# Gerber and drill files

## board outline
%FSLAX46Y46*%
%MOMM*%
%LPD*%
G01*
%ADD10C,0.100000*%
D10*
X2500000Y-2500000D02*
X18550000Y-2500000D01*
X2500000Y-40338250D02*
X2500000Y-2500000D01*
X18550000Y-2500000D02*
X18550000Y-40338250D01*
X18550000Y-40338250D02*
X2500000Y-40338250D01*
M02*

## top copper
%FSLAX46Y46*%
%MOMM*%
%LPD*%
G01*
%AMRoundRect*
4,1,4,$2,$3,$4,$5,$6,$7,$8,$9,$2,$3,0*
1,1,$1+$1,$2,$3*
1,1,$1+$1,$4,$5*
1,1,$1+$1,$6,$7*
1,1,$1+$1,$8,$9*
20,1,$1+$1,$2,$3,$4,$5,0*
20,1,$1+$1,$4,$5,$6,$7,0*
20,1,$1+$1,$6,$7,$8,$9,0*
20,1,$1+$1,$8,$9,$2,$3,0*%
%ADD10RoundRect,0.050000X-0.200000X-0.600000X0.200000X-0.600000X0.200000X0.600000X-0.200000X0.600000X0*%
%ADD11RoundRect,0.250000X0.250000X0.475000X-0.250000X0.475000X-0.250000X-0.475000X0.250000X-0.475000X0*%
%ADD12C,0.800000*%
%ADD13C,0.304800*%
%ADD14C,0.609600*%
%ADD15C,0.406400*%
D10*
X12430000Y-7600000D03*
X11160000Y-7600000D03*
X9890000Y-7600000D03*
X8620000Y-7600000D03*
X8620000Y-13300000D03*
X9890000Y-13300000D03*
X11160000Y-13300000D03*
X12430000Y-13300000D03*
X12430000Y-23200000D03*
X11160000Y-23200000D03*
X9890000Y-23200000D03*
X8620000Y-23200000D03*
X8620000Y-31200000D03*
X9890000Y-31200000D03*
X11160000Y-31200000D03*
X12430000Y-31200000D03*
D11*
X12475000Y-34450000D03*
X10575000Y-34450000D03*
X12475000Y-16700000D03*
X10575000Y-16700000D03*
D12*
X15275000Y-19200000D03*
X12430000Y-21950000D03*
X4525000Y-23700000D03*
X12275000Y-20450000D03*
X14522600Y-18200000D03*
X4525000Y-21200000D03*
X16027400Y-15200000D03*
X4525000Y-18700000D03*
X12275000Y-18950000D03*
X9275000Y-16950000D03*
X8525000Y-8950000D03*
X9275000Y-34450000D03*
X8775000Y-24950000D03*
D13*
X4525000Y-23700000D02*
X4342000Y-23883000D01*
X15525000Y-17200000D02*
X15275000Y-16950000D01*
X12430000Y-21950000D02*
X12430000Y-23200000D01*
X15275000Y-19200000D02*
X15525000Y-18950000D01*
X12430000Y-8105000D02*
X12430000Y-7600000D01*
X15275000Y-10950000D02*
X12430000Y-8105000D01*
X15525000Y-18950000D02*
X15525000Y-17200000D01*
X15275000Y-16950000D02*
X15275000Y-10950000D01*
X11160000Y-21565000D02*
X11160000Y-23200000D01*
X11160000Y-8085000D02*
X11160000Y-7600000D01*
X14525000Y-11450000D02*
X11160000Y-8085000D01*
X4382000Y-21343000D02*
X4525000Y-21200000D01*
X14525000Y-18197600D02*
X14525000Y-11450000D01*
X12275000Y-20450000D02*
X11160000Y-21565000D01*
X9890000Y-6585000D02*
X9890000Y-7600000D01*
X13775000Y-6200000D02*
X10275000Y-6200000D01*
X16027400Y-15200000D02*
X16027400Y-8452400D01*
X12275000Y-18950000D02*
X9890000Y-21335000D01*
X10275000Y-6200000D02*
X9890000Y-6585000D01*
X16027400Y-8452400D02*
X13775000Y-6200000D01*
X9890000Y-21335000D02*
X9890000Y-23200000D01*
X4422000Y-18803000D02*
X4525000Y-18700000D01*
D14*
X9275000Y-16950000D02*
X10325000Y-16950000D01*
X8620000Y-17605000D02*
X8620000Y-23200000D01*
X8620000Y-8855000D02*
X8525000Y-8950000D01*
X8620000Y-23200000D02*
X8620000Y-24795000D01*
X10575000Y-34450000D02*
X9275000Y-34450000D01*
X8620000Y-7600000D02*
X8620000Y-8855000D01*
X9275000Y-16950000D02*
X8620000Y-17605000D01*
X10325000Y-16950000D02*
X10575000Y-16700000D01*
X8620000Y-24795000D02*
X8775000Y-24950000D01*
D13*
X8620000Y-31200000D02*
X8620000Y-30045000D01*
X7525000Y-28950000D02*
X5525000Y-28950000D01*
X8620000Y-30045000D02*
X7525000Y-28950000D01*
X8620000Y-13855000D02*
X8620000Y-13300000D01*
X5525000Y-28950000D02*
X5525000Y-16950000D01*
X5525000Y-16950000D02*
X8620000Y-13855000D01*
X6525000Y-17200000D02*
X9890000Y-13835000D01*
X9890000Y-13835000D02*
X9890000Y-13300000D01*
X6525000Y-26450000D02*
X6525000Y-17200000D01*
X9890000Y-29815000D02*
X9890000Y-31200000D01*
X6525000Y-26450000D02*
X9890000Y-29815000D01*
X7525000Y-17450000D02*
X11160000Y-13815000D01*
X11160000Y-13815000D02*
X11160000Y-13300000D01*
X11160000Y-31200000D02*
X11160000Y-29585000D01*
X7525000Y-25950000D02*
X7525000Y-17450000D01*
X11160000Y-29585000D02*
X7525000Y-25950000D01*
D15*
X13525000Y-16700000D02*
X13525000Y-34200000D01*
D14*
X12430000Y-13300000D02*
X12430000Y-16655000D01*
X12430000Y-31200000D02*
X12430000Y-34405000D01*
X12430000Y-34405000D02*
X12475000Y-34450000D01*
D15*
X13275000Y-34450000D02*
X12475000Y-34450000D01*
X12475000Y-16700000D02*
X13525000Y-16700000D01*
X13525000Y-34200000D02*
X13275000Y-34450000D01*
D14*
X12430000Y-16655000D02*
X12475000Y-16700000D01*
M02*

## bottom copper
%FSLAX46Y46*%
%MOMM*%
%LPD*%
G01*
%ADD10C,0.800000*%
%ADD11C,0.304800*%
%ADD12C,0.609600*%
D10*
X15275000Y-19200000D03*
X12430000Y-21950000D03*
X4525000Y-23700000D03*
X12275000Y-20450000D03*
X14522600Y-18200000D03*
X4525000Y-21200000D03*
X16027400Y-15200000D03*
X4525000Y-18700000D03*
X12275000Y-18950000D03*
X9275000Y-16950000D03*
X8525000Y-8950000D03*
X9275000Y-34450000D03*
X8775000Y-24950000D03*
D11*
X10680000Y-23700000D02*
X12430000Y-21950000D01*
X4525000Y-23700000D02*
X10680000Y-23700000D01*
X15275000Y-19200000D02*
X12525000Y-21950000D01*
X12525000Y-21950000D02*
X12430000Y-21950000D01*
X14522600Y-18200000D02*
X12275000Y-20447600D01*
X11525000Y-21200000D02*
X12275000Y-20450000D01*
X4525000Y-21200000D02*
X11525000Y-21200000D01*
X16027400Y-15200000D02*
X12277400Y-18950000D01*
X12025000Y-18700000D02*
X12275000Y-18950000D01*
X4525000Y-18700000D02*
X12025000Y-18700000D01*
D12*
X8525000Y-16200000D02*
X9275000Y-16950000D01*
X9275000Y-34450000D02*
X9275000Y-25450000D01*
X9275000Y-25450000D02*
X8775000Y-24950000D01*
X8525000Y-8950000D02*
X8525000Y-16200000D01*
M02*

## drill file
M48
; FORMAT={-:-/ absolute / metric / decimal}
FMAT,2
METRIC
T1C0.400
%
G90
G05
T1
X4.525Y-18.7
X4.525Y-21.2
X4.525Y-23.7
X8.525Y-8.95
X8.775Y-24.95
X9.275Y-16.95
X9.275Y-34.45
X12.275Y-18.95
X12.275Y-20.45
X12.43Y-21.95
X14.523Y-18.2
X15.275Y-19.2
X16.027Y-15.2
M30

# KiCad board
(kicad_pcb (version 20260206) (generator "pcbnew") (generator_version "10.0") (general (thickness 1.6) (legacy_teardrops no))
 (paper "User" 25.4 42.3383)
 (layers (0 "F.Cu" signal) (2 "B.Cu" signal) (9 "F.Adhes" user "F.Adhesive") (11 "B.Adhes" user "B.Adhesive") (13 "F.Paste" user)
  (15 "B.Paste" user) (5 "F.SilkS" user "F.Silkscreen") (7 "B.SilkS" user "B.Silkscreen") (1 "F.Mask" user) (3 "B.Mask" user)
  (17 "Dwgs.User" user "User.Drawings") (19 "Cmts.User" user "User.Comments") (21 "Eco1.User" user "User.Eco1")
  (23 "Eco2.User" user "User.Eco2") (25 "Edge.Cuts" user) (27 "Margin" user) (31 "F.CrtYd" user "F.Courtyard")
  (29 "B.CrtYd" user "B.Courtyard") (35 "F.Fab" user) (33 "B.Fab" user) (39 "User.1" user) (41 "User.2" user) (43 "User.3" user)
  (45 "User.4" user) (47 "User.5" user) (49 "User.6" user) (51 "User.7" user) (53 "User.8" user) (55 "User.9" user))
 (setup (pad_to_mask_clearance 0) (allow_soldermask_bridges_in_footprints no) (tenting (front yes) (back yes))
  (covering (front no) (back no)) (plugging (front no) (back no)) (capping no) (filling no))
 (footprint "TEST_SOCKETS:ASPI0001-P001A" (layer "F.Cu") (at 10.525 10.45)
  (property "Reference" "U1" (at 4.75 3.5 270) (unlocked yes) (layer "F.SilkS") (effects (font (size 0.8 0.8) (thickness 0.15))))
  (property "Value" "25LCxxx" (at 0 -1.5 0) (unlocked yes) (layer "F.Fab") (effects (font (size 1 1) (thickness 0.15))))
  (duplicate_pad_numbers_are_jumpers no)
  (pad "1" smd roundrect (at 1.905 -2.85) (size 0.5 1.3) (layers "F.Cu" "F.Mask" "F.Paste") (roundrect_rratio 0.1) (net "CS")
   (thermal_bridge_angle 45))
  (pad "2" smd roundrect (at 0.635 -2.85) (size 0.5 1.3) (layers "F.Cu" "F.Mask" "F.Paste") (roundrect_rratio 0.1) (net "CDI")
   (thermal_bridge_angle 45))
  (pad "3" smd roundrect (at -0.635 -2.85) (size 0.5 1.3) (layers "F.Cu" "F.Mask" "F.Paste") (roundrect_rratio 0.1) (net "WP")
   (thermal_bridge_angle 45))
  (pad "4" smd roundrect (at -1.905 -2.85) (size 0.5 1.3) (layers "F.Cu" "F.Mask" "F.Paste") (roundrect_rratio 0.1) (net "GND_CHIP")
   (thermal_bridge_angle 45))
  (pad "5" smd roundrect (at -1.905 2.85) (size 0.5 1.3) (layers "F.Cu" "F.Mask" "F.Paste") (roundrect_rratio 0.1) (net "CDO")
   (thermal_bridge_angle 45))
  (pad "6" smd roundrect (at -0.635 2.85) (size 0.5 1.3) (layers "F.Cu" "F.Mask" "F.Paste") (roundrect_rratio 0.1) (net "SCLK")
   (thermal_bridge_angle 45))
  (pad "7" smd roundrect (at 0.635 2.85) (size 0.5 1.3) (layers "F.Cu" "F.Mask" "F.Paste") (roundrect_rratio 0.1) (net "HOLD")
   (thermal_bridge_angle 45))
  (pad "8" smd roundrect (at 1.905 2.85) (size 0.5 1.3) (layers "F.Cu" "F.Mask" "F.Paste") (roundrect_rratio 0.1) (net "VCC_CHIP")
   (thermal_bridge_angle 45)))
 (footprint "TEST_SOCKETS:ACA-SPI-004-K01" (layer "F.Cu") (at 10.525 27.2)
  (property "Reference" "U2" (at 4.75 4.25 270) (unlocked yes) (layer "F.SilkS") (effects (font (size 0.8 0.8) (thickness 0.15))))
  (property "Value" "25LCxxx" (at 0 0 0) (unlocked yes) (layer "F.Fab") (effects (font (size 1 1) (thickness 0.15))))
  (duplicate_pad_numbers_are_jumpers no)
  (pad "1" smd roundrect (at 1.905 -4) (size 0.5 1.3) (layers "F.Cu" "F.Mask" "F.Paste") (roundrect_rratio 0.1) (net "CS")
   (thermal_bridge_angle 45))
  (pad "2" smd roundrect (at 0.635 -4) (size 0.5 1.3) (layers "F.Cu" "F.Mask" "F.Paste") (roundrect_rratio 0.1) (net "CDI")
   (thermal_bridge_angle 45))
  (pad "3" smd roundrect (at -0.635 -4) (size 0.5 1.3) (layers "F.Cu" "F.Mask" "F.Paste") (roundrect_rratio 0.1) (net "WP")
   (thermal_bridge_angle 45))
  (pad "4" smd roundrect (at -1.905 -4) (size 0.5 1.3) (layers "F.Cu" "F.Mask" "F.Paste") (roundrect_rratio 0.1) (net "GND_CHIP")
   (thermal_bridge_angle 45))
  (pad "5" smd roundrect (at -1.905 4) (size 0.5 1.3) (layers "F.Cu" "F.Mask" "F.Paste") (roundrect_rratio 0.1) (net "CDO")
   (thermal_bridge_angle 45))
  (pad "6" smd roundrect (at -0.635 4) (size 0.5 1.3) (layers "F.Cu" "F.Mask" "F.Paste") (roundrect_rratio 0.1) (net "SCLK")
   (thermal_bridge_angle 45))
  (pad "7" smd roundrect (at 0.635 4) (size 0.5 1.3) (layers "F.Cu" "F.Mask" "F.Paste") (roundrect_rratio 0.1) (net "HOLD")
   (thermal_bridge_angle 45))
  (pad "8" smd roundrect (at 1.905 4) (size 0.5 1.3) (layers "F.Cu" "F.Mask" "F.Paste") (roundrect_rratio 0.1) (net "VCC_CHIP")
   (thermal_bridge_angle 45)))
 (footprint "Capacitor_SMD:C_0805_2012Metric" (layer "F.Cu") (at 11.525 34.45 180)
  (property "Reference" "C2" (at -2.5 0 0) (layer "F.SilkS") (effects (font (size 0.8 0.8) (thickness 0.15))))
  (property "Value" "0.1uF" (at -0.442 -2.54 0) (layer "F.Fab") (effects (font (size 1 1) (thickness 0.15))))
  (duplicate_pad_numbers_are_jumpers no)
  (pad "1" smd roundrect (at -0.95 0 180) (size 1 1.45) (layers "F.Cu" "F.Mask" "F.Paste") (roundrect_rratio 0.25) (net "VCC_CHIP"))
  (pad "2" smd roundrect (at 0.95 0 180) (size 1 1.45) (layers "F.Cu" "F.Mask" "F.Paste") (roundrect_rratio 0.25) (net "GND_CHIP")))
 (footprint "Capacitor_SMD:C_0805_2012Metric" (layer "F.Cu") (at 11.525 16.7 180)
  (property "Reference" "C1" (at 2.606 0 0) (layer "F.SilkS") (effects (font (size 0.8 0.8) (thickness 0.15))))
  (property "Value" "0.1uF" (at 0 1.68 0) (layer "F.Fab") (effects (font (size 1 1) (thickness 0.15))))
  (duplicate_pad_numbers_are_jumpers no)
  (pad "1" smd roundrect (at -0.95 0 180) (size 1 1.45) (layers "F.Cu" "F.Mask" "F.Paste") (roundrect_rratio 0.25) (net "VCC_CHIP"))
  (pad "2" smd roundrect (at 0.95 0 180) (size 1 1.45) (layers "F.Cu" "F.Mask" "F.Paste") (roundrect_rratio 0.25) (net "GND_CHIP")))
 (gr_line (start 2.5 2.5) (end 18.55 2.5) (stroke (width 0.1) (type default)) (layer "Edge.Cuts"))
 (gr_line (start 2.5 40.33825) (end 2.5 2.5) (stroke (width 0.1) (type default)) (layer "Edge.Cuts"))
 (gr_line (start 18.55 2.5) (end 18.55 40.33825) (stroke (width 0.1) (type default)) (layer "Edge.Cuts"))
 (gr_line (start 18.55 40.33825) (end 2.5 40.33825) (stroke (width 0.1) (type default)) (layer "Edge.Cuts"))
 (segment (start 4.525 23.7) (end 4.342 23.883) (width 0.3048) (layer "F.Cu") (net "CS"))
 (segment (start 15.525 17.2) (end 15.275 16.95) (width 0.3048) (layer "F.Cu") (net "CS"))
 (segment (start 12.43 21.95) (end 12.43 23.2) (width 0.3048) (layer "F.Cu") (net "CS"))
 (segment (start 15.275 19.2) (end 15.525 18.95) (width 0.3048) (layer "F.Cu") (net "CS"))
 (segment (start 12.43 8.105) (end 12.43 7.6) (width 0.3048) (layer "F.Cu") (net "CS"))
 (segment (start 15.275 10.95) (end 12.43 8.105) (width 0.3048) (layer "F.Cu") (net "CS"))
 (segment (start 15.525 18.95) (end 15.525 17.2) (width 0.3048) (layer "F.Cu") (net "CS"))
 (segment (start 15.275 16.95) (end 15.275 10.95) (width 0.3048) (layer "F.Cu") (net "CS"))
 (via (at 15.275 19.2) (size 0.8) (drill 0.4) (layers "F.Cu" "B.Cu") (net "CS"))
 (via (at 12.43 21.95) (size 0.8) (drill 0.4) (layers "F.Cu" "B.Cu") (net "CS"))
 (via (at 4.525 23.7) (size 0.8) (drill 0.4) (layers "F.Cu" "B.Cu") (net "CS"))
 (segment (start 10.68 23.7) (end 12.43 21.95) (width 0.3048) (layer "B.Cu") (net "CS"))
 (segment (start 4.525 23.7) (end 10.68 23.7) (width 0.3048) (layer "B.Cu") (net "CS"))
 (segment (start 15.275 19.2) (end 12.525 21.95) (width 0.3048) (layer "B.Cu") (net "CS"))
 (segment (start 12.525 21.95) (end 12.43 21.95) (width 0.3048) (layer "B.Cu") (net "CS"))
 (segment (start 11.16 21.565) (end 11.16 23.2) (width 0.3048) (layer "F.Cu") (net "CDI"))
 (segment (start 11.16 8.085) (end 11.16 7.6) (width 0.3048) (layer "F.Cu") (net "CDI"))
 (segment (start 14.525 11.45) (end 11.16 8.085) (width 0.3048) (layer "F.Cu") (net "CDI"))
 (segment (start 4.382 21.343) (end 4.525 21.2) (width 0.3048) (layer "F.Cu") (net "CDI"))
 (segment (start 14.525 18.1976) (end 14.525 11.45) (width 0.3048) (layer "F.Cu") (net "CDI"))
 (segment (start 12.275 20.45) (end 11.16 21.565) (width 0.3048) (layer "F.Cu") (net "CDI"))
 (via (at 12.275 20.45) (size 0.8) (drill 0.4) (layers "F.Cu" "B.Cu") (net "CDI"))
 (via (at 14.5226 18.2) (size 0.8) (drill 0.4) (layers "F.Cu" "B.Cu") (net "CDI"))
 (via (at 4.525 21.2) (size 0.8) (drill 0.4) (layers "F.Cu" "B.Cu") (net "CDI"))
 (segment (start 14.5226 18.2) (end 12.275 20.4476) (width 0.3048) (layer "B.Cu") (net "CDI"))
 (segment (start 11.525 21.2) (end 12.275 20.45) (width 0.3048) (layer "B.Cu") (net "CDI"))
 (segment (start 4.525 21.2) (end 11.525 21.2) (width 0.3048) (layer "B.Cu") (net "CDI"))
 (segment (start 9.89 6.585) (end 9.89 7.6) (width 0.3048) (layer "F.Cu") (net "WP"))
 (segment (start 13.775 6.2) (end 10.275 6.2) (width 0.3048) (layer "F.Cu") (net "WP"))
 (segment (start 16.0274 15.2) (end 16.0274 8.4524) (width 0.3048) (layer "F.Cu") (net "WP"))
 (segment (start 12.275 18.95) (end 9.89 21.335) (width 0.3048) (layer "F.Cu") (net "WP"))
 (segment (start 10.275 6.2) (end 9.89 6.585) (width 0.3048) (layer "F.Cu") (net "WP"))
 (segment (start 16.0274 8.4524) (end 13.775 6.2) (width 0.3048) (layer "F.Cu") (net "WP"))
 (segment (start 9.89 21.335) (end 9.89 23.2) (width 0.3048) (layer "F.Cu") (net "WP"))
 (segment (start 4.422 18.803) (end 4.525 18.7) (width 0.3048) (layer "F.Cu") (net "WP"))
 (via (at 16.0274 15.2) (size 0.8) (drill 0.4) (layers "F.Cu" "B.Cu") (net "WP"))
 (via (at 4.525 18.7) (size 0.8) (drill 0.4) (layers "F.Cu" "B.Cu") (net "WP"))
 (via (at 12.275 18.95) (size 0.8) (drill 0.4) (layers "F.Cu" "B.Cu") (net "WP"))
 (segment (start 16.0274 15.2) (end 12.2774 18.95) (width 0.3048) (layer "B.Cu") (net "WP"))
 (segment (start 12.025 18.7) (end 12.275 18.95) (width 0.3048) (layer "B.Cu") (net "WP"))
 (segment (start 4.525 18.7) (end 12.025 18.7) (width 0.3048) (layer "B.Cu") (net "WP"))
 (segment (start 9.275 16.95) (end 10.325 16.95) (width 0.6096) (layer "F.Cu") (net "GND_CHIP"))
 (segment (start 8.62 17.605) (end 8.62 23.2) (width 0.6096) (layer "F.Cu") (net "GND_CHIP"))
 (segment (start 8.62 8.855) (end 8.525 8.95) (width 0.6096) (layer "F.Cu") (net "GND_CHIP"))
 (segment (start 8.62 23.2) (end 8.62 24.795) (width 0.6096) (layer "F.Cu") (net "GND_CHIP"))
 (segment (start 10.575 34.45) (end 9.275 34.45) (width 0.6096) (layer "F.Cu") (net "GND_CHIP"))
 (segment (start 8.62 7.6) (end 8.62 8.855) (width 0.6096) (layer "F.Cu") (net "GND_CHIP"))
 (segment (start 9.275 16.95) (end 8.62 17.605) (width 0.6096) (layer "F.Cu") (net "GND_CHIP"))
 (segment (start 10.325 16.95) (end 10.575 16.7) (width 0.6096) (layer "F.Cu") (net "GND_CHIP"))
 (segment (start 8.62 24.795) (end 8.775 24.95) (width 0.6096) (layer "F.Cu") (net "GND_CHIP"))
 (via (at 9.275 16.95) (size 0.8) (drill 0.4) (layers "F.Cu" "B.Cu") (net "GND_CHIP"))
 (via (at 8.525 8.95) (size 0.8) (drill 0.4) (layers "F.Cu" "B.Cu") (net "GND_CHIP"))
 (via (at 9.275 34.45) (size 0.8) (drill 0.4) (layers "F.Cu" "B.Cu") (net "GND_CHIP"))
 (via (at 8.775 24.95) (size 0.8) (drill 0.4) (layers "F.Cu" "B.Cu") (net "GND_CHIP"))
 (segment (start 8.525 16.2) (end 9.275 16.95) (width 0.6096) (layer "B.Cu") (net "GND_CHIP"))
 (segment (start 9.275 34.45) (end 9.275 25.45) (width 0.6096) (layer "B.Cu") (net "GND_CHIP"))
 (segment (start 9.275 25.45) (end 8.775 24.95) (width 0.6096) (layer "B.Cu") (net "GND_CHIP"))
 (segment (start 8.525 8.95) (end 8.525 16.2) (width 0.6096) (layer "B.Cu") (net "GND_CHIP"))
 (segment (start 8.62 31.2) (end 8.62 30.045) (width 0.3048) (layer "F.Cu") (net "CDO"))
 (segment (start 7.525 28.95) (end 5.525 28.95) (width 0.3048) (layer "F.Cu") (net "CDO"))
 (segment (start 8.62 30.045) (end 7.525 28.95) (width 0.3048) (layer "F.Cu") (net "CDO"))
 (segment (start 8.62 13.855) (end 8.62 13.3) (width 0.3048) (layer "F.Cu") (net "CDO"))
 (segment (start 5.525 28.95) (end 5.525 16.95) (width 0.3048) (layer "F.Cu") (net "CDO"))
 (segment (start 5.525 16.95) (end 8.62 13.855) (width 0.3048) (layer "F.Cu") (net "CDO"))
 (segment (start 6.525 17.2) (end 9.89 13.835) (width 0.3048) (layer "F.Cu") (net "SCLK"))
 (segment (start 9.89 13.835) (end 9.89 13.3) (width 0.3048) (layer "F.Cu") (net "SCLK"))
 (segment (start 6.525 26.45) (end 6.525 17.2) (width 0.3048) (layer "F.Cu") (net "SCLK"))
 (segment (start 9.89 29.815) (end 9.89 31.2) (width 0.3048) (layer "F.Cu") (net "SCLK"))
 (segment (start 6.525 26.45) (end 9.89 29.815) (width 0.3048) (layer "F.Cu") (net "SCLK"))
 (segment (start 7.525 17.45) (end 11.16 13.815) (width 0.3048) (layer "F.Cu") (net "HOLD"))
 (segment (start 11.16 13.815) (end 11.16 13.3) (width 0.3048) (layer "F.Cu") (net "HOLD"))
 (segment (start 11.16 31.2) (end 11.16 29.585) (width 0.3048) (layer "F.Cu") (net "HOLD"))
 (segment (start 7.525 25.95) (end 7.525 17.45) (width 0.3048) (layer "F.Cu") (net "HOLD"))
 (segment (start 11.16 29.585) (end 7.525 25.95) (width 0.3048) (layer "F.Cu") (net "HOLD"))
 (segment (start 13.525 16.7) (end 13.525 34.2) (width 0.4064) (layer "F.Cu") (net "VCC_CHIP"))
 (segment (start 12.43 13.3) (end 12.43 16.655) (width 0.6096) (layer "F.Cu") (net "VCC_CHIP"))
 (segment (start 12.43 31.2) (end 12.43 34.405) (width 0.6096) (layer "F.Cu") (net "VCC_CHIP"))
 (segment (start 12.43 34.405) (end 12.475 34.45) (width 0.6096) (layer "F.Cu") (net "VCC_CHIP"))
 (segment (start 13.275 34.45) (end 12.475 34.45) (width 0.4064) (layer "F.Cu") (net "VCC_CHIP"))
 (segment (start 12.475 16.7) (end 13.525 16.7) (width 0.4064) (layer "F.Cu") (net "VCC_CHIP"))
 (segment (start 13.525 34.2) (end 13.275 34.45) (width 0.4064) (layer "F.Cu") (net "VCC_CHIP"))
 (segment (start 12.43 16.655) (end 12.475 16.7) (width 0.6096) (layer "F.Cu") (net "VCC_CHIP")))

